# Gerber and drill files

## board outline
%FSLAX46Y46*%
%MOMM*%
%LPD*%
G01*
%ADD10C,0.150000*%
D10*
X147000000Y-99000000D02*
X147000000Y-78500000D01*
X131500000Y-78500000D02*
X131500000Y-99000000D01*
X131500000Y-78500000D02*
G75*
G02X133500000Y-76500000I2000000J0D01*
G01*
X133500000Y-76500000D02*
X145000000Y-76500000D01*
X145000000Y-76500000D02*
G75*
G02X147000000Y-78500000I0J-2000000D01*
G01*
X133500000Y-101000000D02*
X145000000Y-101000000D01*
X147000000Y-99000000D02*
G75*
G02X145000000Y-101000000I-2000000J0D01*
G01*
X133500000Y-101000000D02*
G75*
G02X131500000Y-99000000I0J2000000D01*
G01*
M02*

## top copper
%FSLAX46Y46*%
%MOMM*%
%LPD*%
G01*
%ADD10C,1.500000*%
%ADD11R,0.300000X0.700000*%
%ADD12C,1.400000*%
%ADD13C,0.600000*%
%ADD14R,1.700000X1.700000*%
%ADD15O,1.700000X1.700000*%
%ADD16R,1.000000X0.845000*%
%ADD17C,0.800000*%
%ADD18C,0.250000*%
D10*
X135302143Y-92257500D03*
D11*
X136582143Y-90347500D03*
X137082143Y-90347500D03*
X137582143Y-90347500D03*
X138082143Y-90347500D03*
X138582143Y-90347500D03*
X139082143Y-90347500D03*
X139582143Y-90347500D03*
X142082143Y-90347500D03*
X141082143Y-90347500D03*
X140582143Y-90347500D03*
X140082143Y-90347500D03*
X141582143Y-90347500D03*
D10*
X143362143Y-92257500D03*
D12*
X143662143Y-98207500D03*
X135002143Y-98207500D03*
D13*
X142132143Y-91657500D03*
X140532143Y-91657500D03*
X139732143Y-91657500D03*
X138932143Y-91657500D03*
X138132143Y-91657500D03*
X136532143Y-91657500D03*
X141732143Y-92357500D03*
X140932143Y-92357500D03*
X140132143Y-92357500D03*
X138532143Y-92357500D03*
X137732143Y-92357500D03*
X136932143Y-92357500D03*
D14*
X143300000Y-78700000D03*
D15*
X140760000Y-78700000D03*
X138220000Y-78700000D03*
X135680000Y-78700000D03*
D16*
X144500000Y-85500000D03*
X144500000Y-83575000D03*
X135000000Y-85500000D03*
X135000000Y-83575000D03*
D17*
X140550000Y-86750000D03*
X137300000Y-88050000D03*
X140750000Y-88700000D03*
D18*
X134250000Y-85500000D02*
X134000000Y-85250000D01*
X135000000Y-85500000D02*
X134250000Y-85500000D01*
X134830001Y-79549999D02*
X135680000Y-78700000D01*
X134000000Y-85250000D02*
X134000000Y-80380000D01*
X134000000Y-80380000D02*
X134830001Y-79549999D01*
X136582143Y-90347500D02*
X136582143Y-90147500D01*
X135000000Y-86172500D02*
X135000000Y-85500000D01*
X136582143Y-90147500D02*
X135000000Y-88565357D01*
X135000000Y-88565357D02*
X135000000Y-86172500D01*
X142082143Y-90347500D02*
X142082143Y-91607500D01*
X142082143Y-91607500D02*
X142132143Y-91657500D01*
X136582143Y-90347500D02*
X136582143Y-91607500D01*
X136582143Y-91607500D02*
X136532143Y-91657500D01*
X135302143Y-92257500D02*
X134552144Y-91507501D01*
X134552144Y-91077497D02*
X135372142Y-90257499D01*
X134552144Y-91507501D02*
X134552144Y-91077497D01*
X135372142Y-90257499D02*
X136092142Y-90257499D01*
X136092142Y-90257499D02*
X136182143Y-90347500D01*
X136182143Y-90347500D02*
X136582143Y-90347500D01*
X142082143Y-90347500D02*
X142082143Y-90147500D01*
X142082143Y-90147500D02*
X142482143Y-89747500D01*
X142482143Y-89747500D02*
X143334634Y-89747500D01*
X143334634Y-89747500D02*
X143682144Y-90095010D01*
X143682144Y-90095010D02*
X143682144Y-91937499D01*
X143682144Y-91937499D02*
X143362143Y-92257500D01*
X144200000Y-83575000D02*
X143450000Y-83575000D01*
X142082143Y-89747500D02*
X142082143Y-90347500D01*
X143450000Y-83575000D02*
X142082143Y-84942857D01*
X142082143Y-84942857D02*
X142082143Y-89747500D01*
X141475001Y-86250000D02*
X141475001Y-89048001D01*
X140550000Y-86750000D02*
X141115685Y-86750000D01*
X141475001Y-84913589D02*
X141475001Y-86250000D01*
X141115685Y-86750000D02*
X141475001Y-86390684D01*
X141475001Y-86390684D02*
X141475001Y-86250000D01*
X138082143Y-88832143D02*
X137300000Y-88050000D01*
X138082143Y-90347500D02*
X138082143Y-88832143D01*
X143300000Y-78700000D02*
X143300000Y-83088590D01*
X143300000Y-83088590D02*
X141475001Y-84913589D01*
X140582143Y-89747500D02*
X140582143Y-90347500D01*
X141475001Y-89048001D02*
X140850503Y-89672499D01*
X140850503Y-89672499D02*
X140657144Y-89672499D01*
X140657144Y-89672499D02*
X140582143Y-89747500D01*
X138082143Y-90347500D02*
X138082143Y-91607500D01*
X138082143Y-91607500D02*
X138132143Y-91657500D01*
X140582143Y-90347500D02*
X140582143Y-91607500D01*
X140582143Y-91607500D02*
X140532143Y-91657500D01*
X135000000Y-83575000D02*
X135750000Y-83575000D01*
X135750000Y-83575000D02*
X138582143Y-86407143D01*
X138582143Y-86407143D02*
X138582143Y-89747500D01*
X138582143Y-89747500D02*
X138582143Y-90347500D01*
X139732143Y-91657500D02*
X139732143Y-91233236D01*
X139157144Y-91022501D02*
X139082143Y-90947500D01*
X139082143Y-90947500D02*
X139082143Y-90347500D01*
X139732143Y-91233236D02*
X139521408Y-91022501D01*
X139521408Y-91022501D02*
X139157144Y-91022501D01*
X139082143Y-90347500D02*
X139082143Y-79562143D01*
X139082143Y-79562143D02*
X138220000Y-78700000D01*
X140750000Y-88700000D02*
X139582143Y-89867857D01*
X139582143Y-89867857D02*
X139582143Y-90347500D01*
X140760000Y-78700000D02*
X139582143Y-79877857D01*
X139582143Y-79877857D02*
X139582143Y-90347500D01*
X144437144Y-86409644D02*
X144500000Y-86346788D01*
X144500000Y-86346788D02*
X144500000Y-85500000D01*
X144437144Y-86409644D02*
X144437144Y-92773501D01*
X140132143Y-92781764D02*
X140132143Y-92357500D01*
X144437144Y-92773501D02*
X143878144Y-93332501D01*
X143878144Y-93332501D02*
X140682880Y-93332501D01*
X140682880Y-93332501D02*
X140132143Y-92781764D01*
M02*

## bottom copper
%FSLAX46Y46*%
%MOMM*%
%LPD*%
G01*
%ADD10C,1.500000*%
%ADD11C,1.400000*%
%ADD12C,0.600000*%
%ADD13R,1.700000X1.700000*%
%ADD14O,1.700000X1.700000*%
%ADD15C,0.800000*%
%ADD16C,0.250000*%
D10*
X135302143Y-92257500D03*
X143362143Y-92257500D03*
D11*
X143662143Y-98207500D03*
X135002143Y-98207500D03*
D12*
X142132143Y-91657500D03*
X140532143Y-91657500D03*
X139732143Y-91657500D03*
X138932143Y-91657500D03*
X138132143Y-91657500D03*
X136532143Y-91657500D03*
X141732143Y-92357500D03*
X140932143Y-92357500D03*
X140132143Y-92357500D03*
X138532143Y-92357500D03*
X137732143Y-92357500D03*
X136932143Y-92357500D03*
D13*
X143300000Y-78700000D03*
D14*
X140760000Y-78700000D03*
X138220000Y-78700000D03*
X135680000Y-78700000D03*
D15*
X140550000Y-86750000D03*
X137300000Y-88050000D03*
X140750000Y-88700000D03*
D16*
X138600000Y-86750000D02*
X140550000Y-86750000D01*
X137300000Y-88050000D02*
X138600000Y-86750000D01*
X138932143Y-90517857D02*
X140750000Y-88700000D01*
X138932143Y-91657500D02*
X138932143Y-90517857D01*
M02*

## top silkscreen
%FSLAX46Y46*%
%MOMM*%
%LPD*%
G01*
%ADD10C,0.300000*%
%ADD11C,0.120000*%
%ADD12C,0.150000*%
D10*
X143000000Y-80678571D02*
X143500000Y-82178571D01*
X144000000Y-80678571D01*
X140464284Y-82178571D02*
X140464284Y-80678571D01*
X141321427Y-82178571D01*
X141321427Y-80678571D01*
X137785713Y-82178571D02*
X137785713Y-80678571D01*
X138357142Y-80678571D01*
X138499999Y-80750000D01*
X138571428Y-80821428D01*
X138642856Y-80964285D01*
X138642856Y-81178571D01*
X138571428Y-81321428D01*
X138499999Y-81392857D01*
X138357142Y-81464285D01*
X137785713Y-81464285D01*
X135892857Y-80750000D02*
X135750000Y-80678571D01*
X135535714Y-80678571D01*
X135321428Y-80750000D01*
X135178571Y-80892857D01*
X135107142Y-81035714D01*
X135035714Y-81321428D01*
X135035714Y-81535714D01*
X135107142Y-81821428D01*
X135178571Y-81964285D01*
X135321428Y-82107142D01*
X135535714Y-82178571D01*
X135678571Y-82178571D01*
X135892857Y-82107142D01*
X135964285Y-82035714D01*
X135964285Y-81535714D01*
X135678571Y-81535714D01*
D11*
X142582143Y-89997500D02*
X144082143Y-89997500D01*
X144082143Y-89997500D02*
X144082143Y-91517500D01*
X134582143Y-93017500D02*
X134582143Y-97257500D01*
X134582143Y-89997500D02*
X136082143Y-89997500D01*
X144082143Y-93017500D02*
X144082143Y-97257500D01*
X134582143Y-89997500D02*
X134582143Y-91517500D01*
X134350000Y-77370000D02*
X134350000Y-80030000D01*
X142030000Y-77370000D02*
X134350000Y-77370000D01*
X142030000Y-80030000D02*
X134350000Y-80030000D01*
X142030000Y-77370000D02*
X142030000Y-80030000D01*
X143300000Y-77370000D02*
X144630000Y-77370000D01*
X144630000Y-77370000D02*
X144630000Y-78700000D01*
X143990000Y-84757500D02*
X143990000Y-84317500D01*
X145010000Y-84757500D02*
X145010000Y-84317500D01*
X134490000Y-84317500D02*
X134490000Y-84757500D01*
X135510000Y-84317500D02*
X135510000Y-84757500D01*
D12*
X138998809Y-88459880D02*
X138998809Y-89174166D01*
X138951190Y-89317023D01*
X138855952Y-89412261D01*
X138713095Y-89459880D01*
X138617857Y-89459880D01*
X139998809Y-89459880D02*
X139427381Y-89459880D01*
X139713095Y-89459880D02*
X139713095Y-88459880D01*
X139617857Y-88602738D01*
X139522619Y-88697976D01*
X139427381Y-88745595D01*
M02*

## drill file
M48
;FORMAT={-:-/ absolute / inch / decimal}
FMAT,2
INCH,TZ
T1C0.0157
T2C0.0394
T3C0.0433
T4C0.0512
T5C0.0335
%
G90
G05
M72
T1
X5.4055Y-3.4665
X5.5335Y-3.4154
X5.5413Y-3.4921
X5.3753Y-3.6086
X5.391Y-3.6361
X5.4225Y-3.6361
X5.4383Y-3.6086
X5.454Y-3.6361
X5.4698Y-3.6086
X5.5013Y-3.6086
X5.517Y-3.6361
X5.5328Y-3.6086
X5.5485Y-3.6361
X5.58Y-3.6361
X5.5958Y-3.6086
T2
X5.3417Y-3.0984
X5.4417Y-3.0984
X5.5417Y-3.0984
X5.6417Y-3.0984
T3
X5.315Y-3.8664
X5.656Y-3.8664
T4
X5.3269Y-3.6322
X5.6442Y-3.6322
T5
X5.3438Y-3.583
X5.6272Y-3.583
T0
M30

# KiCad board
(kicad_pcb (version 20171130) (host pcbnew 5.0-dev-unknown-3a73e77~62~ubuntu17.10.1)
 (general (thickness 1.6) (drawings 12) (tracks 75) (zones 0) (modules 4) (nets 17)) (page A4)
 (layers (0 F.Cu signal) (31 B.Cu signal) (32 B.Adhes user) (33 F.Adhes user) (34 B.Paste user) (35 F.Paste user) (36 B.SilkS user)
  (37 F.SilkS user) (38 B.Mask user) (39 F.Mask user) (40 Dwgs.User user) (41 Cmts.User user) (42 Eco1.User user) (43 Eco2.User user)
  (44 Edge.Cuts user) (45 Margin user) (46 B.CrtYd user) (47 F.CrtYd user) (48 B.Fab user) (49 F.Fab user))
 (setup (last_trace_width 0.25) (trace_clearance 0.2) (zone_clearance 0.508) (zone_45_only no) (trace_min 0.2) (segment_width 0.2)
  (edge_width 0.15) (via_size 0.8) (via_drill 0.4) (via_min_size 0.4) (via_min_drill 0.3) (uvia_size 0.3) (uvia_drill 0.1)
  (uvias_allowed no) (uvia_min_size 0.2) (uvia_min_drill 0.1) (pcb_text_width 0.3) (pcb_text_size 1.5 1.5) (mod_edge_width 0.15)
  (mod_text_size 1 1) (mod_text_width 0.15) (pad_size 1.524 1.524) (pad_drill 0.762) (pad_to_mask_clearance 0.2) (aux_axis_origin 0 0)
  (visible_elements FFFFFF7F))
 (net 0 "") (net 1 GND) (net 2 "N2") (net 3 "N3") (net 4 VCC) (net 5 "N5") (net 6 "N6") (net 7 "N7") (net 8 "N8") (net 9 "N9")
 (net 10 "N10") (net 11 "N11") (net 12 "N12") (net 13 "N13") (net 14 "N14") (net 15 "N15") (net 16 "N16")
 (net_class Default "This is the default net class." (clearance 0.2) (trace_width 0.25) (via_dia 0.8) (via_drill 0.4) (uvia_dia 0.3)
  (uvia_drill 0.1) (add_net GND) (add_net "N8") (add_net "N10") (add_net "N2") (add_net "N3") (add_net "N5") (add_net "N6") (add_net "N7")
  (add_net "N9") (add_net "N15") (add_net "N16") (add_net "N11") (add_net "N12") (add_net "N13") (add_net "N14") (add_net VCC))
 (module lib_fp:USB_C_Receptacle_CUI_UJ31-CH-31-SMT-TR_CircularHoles (layer F.Cu) (at 139.332143 95.3675)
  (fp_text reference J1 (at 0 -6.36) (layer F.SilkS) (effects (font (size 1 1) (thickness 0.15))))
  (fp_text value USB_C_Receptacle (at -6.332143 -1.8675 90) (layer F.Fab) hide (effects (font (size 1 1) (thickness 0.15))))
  (fp_line (start 3.25 -5.37) (end 4.75 -5.37) (layer F.SilkS) (width 0.12))
  (fp_line (start 4.75 -5.37) (end 4.75 -3.85) (layer F.SilkS) (width 0.12))
  (fp_line (start -4.75 -2.35) (end -4.75 1.89) (layer F.SilkS) (width 0.12))
  (fp_line (start -4.75 -5.37) (end -3.25 -5.37) (layer F.SilkS) (width 0.12))
  (fp_line (start 4.75 -2.35) (end 4.75 1.89) (layer F.SilkS) (width 0.12))
  (fp_line (start -4.75 -5.37) (end -4.75 -3.85) (layer F.SilkS) (width 0.12))
  (pad S1 thru_hole circle (at -4.03 -3.11) (size 1.5 1.5) (drill 1.3) (layers *.Cu *.Mask) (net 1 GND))
  (pad A1 smd rect (at -2.75 -5.02) (size 0.3 0.7) (layers F.Cu F.Paste F.Mask) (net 1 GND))
  (pad A2 smd rect (at -2.25 -5.02) (size 0.3 0.7) (layers F.Cu F.Paste F.Mask) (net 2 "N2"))
  (pad A3 smd rect (at -1.75 -5.02) (size 0.3 0.7) (layers F.Cu F.Paste F.Mask) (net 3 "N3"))
  (pad A4 smd rect (at -1.25 -5.02) (size 0.3 0.7) (layers F.Cu F.Paste F.Mask) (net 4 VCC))
  (pad A5 smd rect (at -0.75 -5.02) (size 0.3 0.7) (layers F.Cu F.Paste F.Mask) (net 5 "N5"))
  (pad A6 smd rect (at -0.25 -5.02) (size 0.3 0.7) (layers F.Cu F.Paste F.Mask) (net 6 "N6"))
  (pad A7 smd rect (at 0.25 -5.02) (size 0.3 0.7) (layers F.Cu F.Paste F.Mask) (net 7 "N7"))
  (pad A12 smd rect (at 2.75 -5.02) (size 0.3 0.7) (layers F.Cu F.Paste F.Mask) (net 1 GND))
  (pad A10 smd rect (at 1.75 -5.02) (size 0.3 0.7) (layers F.Cu F.Paste F.Mask) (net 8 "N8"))
  (pad A9 smd rect (at 1.25 -5.02) (size 0.3 0.7) (layers F.Cu F.Paste F.Mask) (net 4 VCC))
  (pad A8 smd rect (at 0.75 -5.02) (size 0.3 0.7) (layers F.Cu F.Paste F.Mask) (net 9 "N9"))
  (pad A11 smd rect (at 2.25 -5.02) (size 0.3 0.7) (layers F.Cu F.Paste F.Mask) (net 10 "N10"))
  (pad S1 thru_hole circle (at 4.03 -3.11) (size 1.5 1.5) (drill 1.3) (layers *.Cu *.Mask) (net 1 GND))
  (pad S1 thru_hole circle (at 4.33 2.84) (size 1.4 1.4) (drill 1.1) (layers *.Cu *.Mask) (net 1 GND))
  (pad S1 thru_hole circle (at -4.33 2.84) (size 1.4 1.4) (drill 1.1) (layers *.Cu *.Mask) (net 1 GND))
  (pad "" np_thru_hole circle (at 3.6 -4.36) (size 0.85 0.85) (drill 0.85) (layers *.Cu *.Mask))
  (pad "" np_thru_hole circle (at -3.6 -4.36) (size 0.85 0.85) (drill 0.85) (layers *.Cu *.Mask))
  (pad B1 thru_hole circle (at 2.8 -3.71) (size 0.6 0.6) (drill 0.4) (layers *.Cu *.Mask) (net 1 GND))
  (pad B4 thru_hole circle (at 1.2 -3.71) (size 0.6 0.6) (drill 0.4) (layers *.Cu *.Mask) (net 4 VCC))
  (pad B6 thru_hole circle (at 0.4 -3.71) (size 0.6 0.6) (drill 0.4) (layers *.Cu *.Mask) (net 6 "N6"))
  (pad B7 thru_hole circle (at -0.4 -3.71) (size 0.6 0.6) (drill 0.4) (layers *.Cu *.Mask) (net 7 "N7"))
  (pad B9 thru_hole circle (at -1.2 -3.71) (size 0.6 0.6) (drill 0.4) (layers *.Cu *.Mask) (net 4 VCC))
  (pad B12 thru_hole circle (at -2.8 -3.71) (size 0.6 0.6) (drill 0.4) (layers *.Cu *.Mask) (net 1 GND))
  (pad B2 thru_hole circle (at 2.4 -3.01) (size 0.6 0.6) (drill 0.4) (layers *.Cu *.Mask) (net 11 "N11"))
  (pad B3 thru_hole circle (at 1.6 -3.01) (size 0.6 0.6) (drill 0.4) (layers *.Cu *.Mask) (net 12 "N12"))
  (pad B5 thru_hole circle (at 0.8 -3.01) (size 0.6 0.6) (drill 0.4) (layers *.Cu *.Mask) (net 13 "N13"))
  (pad B8 thru_hole circle (at -0.8 -3.01) (size 0.6 0.6) (drill 0.4) (layers *.Cu *.Mask) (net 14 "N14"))
  (pad B10 thru_hole circle (at -1.6 -3.01) (size 0.6 0.6) (drill 0.4) (layers *.Cu *.Mask) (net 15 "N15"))
  (pad B11 thru_hole circle (at -2.4 -3.01) (size 0.6 0.6) (drill 0.4) (layers *.Cu *.Mask) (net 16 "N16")))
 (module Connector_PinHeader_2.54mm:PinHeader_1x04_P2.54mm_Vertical (layer F.Cu) (at 143.3 78.7 270)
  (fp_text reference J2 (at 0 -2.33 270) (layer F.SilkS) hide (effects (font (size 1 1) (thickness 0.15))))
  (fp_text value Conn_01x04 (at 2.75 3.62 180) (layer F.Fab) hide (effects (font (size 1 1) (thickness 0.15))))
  (fp_line (start -1.33 8.95) (end 1.33 8.95) (layer F.SilkS) (width 0.12))
  (fp_line (start -1.33 1.27) (end -1.33 8.95) (layer F.SilkS) (width 0.12))
  (fp_line (start 1.33 1.27) (end 1.33 8.95) (layer F.SilkS) (width 0.12))
  (fp_line (start -1.33 1.27) (end 1.33 1.27) (layer F.SilkS) (width 0.12))
  (fp_line (start -1.33 0) (end -1.33 -1.33) (layer F.SilkS) (width 0.12))
  (fp_line (start -1.33 -1.33) (end 0 -1.33) (layer F.SilkS) (width 0.12))
  (pad 1 thru_hole rect (at 0 0 270) (size 1.7 1.7) (drill 1) (layers *.Cu *.Mask) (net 4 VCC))
  (pad 2 thru_hole oval (at 0 2.54 270) (size 1.7 1.7) (drill 1) (layers *.Cu *.Mask) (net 7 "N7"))
  (pad 3 thru_hole oval (at 0 5.08 270) (size 1.7 1.7) (drill 1) (layers *.Cu *.Mask) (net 6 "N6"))
  (pad 4 thru_hole oval (at 0 7.62 270) (size 1.7 1.7) (drill 1) (layers *.Cu *.Mask) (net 1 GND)))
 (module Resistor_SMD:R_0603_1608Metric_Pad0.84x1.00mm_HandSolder (layer F.Cu) (at 144.5 84.5375 90)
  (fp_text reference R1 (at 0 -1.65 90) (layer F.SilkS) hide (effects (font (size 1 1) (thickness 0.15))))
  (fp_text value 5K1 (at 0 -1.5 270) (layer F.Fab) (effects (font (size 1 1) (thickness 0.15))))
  (fp_line (start -0.22 -0.51) (end 0.22 -0.51) (layer F.SilkS) (width 0.12))
  (fp_line (start -0.22 0.51) (end 0.22 0.51) (layer F.SilkS) (width 0.12))
  (pad 1 smd rect (at -0.9625 0 90) (size 0.845 1) (layers F.Cu F.Paste F.Mask) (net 13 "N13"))
  (pad 2 smd rect (at 0.9625 0 90) (size 0.845 1) (layers F.Cu F.Paste F.Mask) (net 1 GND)))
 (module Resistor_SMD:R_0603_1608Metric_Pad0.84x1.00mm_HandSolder (layer F.Cu) (at 135 84.5375 270)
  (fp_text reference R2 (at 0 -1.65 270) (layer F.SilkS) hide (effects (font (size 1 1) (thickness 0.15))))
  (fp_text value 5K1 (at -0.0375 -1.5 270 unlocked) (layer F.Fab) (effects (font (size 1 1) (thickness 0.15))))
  (fp_line (start -0.22 0.51) (end 0.22 0.51) (layer F.SilkS) (width 0.12))
  (fp_line (start -0.22 -0.51) (end 0.22 -0.51) (layer F.SilkS) (width 0.12))
  (pad 2 smd rect (at 0.9625 0 270) (size 0.845 1) (layers F.Cu F.Paste F.Mask) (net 1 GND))
  (pad 1 smd rect (at -0.9625 0 270) (size 0.845 1) (layers F.Cu F.Paste F.Mask) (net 5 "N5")))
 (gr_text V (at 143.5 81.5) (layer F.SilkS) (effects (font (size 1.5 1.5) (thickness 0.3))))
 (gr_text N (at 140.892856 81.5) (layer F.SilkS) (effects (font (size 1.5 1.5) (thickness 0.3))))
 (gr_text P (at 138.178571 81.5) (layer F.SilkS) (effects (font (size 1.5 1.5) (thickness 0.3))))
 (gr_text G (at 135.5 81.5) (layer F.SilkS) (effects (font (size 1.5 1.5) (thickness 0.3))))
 (gr_line (start 147 99) (end 147 78.5) (layer Edge.Cuts) (width 0.15))
 (gr_line (start 131.5 78.5) (end 131.5 99) (layer Edge.Cuts) (width 0.15))
 (gr_arc (start 133.5 78.5) (end 133.5 76.5) (angle -90) (layer Edge.Cuts) (width 0.15))
 (gr_line (start 133.5 76.5) (end 145 76.5) (layer Edge.Cuts) (width 0.15))
 (gr_arc (start 145 78.5) (end 147 78.5) (angle -90) (layer Edge.Cuts) (width 0.15))
 (gr_line (start 133.5 101) (end 145 101) (layer Edge.Cuts) (width 0.15))
 (gr_arc (start 145 99) (end 145 101) (angle -90) (layer Edge.Cuts) (width 0.15))
 (gr_arc (start 133.5 99) (end 131.5 99) (angle -90) (layer Edge.Cuts) (width 0.15))
 (segment (start 134.25 85.5) (end 134 85.25) (width 0.25) (layer F.Cu) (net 1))
 (segment (start 135 85.5) (end 134.25 85.5) (width 0.25) (layer F.Cu) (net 1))
 (segment (start 134.830001 79.549999) (end 135.68 78.7) (width 0.25) (layer F.Cu) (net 1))
 (segment (start 134 85.25) (end 134 80.38) (width 0.25) (layer F.Cu) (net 1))
 (segment (start 134 80.38) (end 134.830001 79.549999) (width 0.25) (layer F.Cu) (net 1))
 (segment (start 136.582143 90.3475) (end 136.582143 90.1475) (width 0.25) (layer F.Cu) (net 1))
 (segment (start 135 86.1725) (end 135 85.5) (width 0.25) (layer F.Cu) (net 1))
 (segment (start 136.582143 90.1475) (end 135 88.565357) (width 0.25) (layer F.Cu) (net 1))
 (segment (start 135 88.565357) (end 135 86.1725) (width 0.25) (layer F.Cu) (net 1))
 (segment (start 142.082143 90.3475) (end 142.082143 91.6075) (width 0.25) (layer F.Cu) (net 1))
 (segment (start 142.082143 91.6075) (end 142.132143 91.6575) (width 0.25) (layer F.Cu) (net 1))
 (segment (start 136.582143 90.3475) (end 136.582143 91.6075) (width 0.25) (layer F.Cu) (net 1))
 (segment (start 136.582143 91.6075) (end 136.532143 91.6575) (width 0.25) (layer F.Cu) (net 1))
 (segment (start 135.302143 92.2575) (end 134.552144 91.507501) (width 0.25) (layer F.Cu) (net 1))
 (segment (start 134.552144 91.077497) (end 135.372142 90.257499) (width 0.25) (layer F.Cu) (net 1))
 (segment (start 134.552144 91.507501) (end 134.552144 91.077497) (width 0.25) (layer F.Cu) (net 1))
 (segment (start 135.372142 90.257499) (end 136.092142 90.257499) (width 0.25) (layer F.Cu) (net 1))
 (segment (start 136.092142 90.257499) (end 136.182143 90.3475) (width 0.25) (layer F.Cu) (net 1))
 (segment (start 136.182143 90.3475) (end 136.582143 90.3475) (width 0.25) (layer F.Cu) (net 1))
 (segment (start 142.082143 90.3475) (end 142.082143 90.1475) (width 0.25) (layer F.Cu) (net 1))
 (segment (start 142.082143 90.1475) (end 142.482143 89.7475) (width 0.25) (layer F.Cu) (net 1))
 (segment (start 142.482143 89.7475) (end 143.334634 89.7475) (width 0.25) (layer F.Cu) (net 1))
 (segment (start 143.334634 89.7475) (end 143.682144 90.09501) (width 0.25) (layer F.Cu) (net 1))
 (segment (start 143.682144 90.09501) (end 143.682144 91.937499) (width 0.25) (layer F.Cu) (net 1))
 (segment (start 143.682144 91.937499) (end 143.362143 92.2575) (width 0.25) (layer F.Cu) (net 1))
 (segment (start 144.2 83.575) (end 143.45 83.575) (width 0.25) (layer F.Cu) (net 1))
 (segment (start 142.082143 89.7475) (end 142.082143 90.3475) (width 0.25) (layer F.Cu) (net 1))
 (segment (start 143.45 83.575) (end 142.082143 84.942857) (width 0.25) (layer F.Cu) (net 1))
 (segment (start 142.082143 84.942857) (end 142.082143 89.7475) (width 0.25) (layer F.Cu) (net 1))
 (segment (start 141.475001 86.25) (end 141.475001 89.048001) (width 0.25) (layer F.Cu) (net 4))
 (segment (start 140.55 86.75) (end 141.115685 86.75) (width 0.25) (layer F.Cu) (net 4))
 (segment (start 141.475001 84.913589) (end 141.475001 86.25) (width 0.25) (layer F.Cu) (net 4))
 (segment (start 141.115685 86.75) (end 141.475001 86.390684) (width 0.25) (layer F.Cu) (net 4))
 (segment (start 141.475001 86.390684) (end 141.475001 86.25) (width 0.25) (layer F.Cu) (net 4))
 (segment (start 138.6 86.75) (end 140.55 86.75) (width 0.25) (layer B.Cu) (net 4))
 (segment (start 137.3 88.05) (end 138.6 86.75) (width 0.25) (layer B.Cu) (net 4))
 (via (at 140.55 86.75) (size 0.8) (drill 0.4) (layers F.Cu B.Cu) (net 4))
 (segment (start 138.082143 88.832143) (end 137.3 88.05) (width 0.25) (layer F.Cu) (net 4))
 (segment (start 138.082143 90.3475) (end 138.082143 88.832143) (width 0.25) (layer F.Cu) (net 4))
 (via (at 137.3 88.05) (size 0.8) (drill 0.4) (layers F.Cu B.Cu) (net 4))
 (segment (start 143.3 78.7) (end 143.3 83.08859) (width 0.25) (layer F.Cu) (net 4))
 (segment (start 143.3 83.08859) (end 141.475001 84.913589) (width 0.25) (layer F.Cu) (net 4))
 (segment (start 140.582143 89.7475) (end 140.582143 90.3475) (width 0.25) (layer F.Cu) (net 4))
 (segment (start 141.475001 89.048001) (end 140.850503 89.672499) (width 0.25) (layer F.Cu) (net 4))
 (segment (start 140.850503 89.672499) (end 140.657144 89.672499) (width 0.25) (layer F.Cu) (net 4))
 (segment (start 140.657144 89.672499) (end 140.582143 89.7475) (width 0.25) (layer F.Cu) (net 4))
 (segment (start 138.082143 90.3475) (end 138.082143 91.6075) (width 0.25) (layer F.Cu) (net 4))
 (segment (start 138.082143 91.6075) (end 138.132143 91.6575) (width 0.25) (layer F.Cu) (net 4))
 (segment (start 140.582143 90.3475) (end 140.582143 91.6075) (width 0.25) (layer F.Cu) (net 4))
 (segment (start 140.582143 91.6075) (end 140.532143 91.6575) (width 0.25) (layer F.Cu) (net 4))
 (segment (start 135 83.575) (end 135.75 83.575) (width 0.25) (layer F.Cu) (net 5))
 (segment (start 135.75 83.575) (end 138.582143 86.407143) (width 0.25) (layer F.Cu) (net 5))
 (segment (start 138.582143 86.407143) (end 138.582143 89.7475) (width 0.25) (layer F.Cu) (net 5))
 (segment (start 138.582143 89.7475) (end 138.582143 90.3475) (width 0.25) (layer F.Cu) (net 5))
 (segment (start 139.732143 91.6575) (end 139.732143 91.233236) (width 0.25) (layer F.Cu) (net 6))
 (segment (start 139.157144 91.022501) (end 139.082143 90.9475) (width 0.25) (layer F.Cu) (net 6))
 (segment (start 139.082143 90.9475) (end 139.082143 90.3475) (width 0.25) (layer F.Cu) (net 6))
 (segment (start 139.732143 91.233236) (end 139.521408 91.022501) (width 0.25) (layer F.Cu) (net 6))
 (segment (start 139.521408 91.022501) (end 139.157144 91.022501) (width 0.25) (layer F.Cu) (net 6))
 (segment (start 139.082143 90.3475) (end 139.082143 79.562143) (width 0.25) (layer F.Cu) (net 6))
 (segment (start 139.082143 79.562143) (end 138.22 78.7) (width 0.25) (layer F.Cu) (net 6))
 (segment (start 140.75 88.7) (end 139.582143 89.867857) (width 0.25) (layer F.Cu) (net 7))
 (segment (start 139.582143 89.867857) (end 139.582143 90.3475) (width 0.25) (layer F.Cu) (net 7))
 (segment (start 138.932143 90.517857) (end 140.75 88.7) (width 0.25) (layer B.Cu) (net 7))
 (segment (start 138.932143 91.6575) (end 138.932143 90.517857) (width 0.25) (layer B.Cu) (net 7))
 (via (at 140.75 88.7) (size 0.8) (drill 0.4) (layers F.Cu B.Cu) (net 7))
 (segment (start 140.76 78.7) (end 139.582143 79.877857) (width 0.25) (layer F.Cu) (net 7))
 (segment (start 139.582143 79.877857) (end 139.582143 90.3475) (width 0.25) (layer F.Cu) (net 7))
 (segment (start 144.437144 86.409644) (end 144.5 86.346788) (width 0.25) (layer F.Cu) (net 13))
 (segment (start 144.5 86.346788) (end 144.5 85.5) (width 0.25) (layer F.Cu) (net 13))
 (segment (start 144.437144 86.409644) (end 144.437144 92.773501) (width 0.25) (layer F.Cu) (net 13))
 (segment (start 140.132143 92.781764) (end 140.132143 92.3575) (width 0.25) (layer F.Cu) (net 13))
 (segment (start 144.437144 92.773501) (end 143.878144 93.332501) (width 0.25) (layer F.Cu) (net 13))
 (segment (start 143.878144 93.332501) (end 140.68288 93.332501) (width 0.25) (layer F.Cu) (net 13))
 (segment (start 140.68288 93.332501) (end 140.132143 92.781764) (width 0.25) (layer F.Cu) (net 13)))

